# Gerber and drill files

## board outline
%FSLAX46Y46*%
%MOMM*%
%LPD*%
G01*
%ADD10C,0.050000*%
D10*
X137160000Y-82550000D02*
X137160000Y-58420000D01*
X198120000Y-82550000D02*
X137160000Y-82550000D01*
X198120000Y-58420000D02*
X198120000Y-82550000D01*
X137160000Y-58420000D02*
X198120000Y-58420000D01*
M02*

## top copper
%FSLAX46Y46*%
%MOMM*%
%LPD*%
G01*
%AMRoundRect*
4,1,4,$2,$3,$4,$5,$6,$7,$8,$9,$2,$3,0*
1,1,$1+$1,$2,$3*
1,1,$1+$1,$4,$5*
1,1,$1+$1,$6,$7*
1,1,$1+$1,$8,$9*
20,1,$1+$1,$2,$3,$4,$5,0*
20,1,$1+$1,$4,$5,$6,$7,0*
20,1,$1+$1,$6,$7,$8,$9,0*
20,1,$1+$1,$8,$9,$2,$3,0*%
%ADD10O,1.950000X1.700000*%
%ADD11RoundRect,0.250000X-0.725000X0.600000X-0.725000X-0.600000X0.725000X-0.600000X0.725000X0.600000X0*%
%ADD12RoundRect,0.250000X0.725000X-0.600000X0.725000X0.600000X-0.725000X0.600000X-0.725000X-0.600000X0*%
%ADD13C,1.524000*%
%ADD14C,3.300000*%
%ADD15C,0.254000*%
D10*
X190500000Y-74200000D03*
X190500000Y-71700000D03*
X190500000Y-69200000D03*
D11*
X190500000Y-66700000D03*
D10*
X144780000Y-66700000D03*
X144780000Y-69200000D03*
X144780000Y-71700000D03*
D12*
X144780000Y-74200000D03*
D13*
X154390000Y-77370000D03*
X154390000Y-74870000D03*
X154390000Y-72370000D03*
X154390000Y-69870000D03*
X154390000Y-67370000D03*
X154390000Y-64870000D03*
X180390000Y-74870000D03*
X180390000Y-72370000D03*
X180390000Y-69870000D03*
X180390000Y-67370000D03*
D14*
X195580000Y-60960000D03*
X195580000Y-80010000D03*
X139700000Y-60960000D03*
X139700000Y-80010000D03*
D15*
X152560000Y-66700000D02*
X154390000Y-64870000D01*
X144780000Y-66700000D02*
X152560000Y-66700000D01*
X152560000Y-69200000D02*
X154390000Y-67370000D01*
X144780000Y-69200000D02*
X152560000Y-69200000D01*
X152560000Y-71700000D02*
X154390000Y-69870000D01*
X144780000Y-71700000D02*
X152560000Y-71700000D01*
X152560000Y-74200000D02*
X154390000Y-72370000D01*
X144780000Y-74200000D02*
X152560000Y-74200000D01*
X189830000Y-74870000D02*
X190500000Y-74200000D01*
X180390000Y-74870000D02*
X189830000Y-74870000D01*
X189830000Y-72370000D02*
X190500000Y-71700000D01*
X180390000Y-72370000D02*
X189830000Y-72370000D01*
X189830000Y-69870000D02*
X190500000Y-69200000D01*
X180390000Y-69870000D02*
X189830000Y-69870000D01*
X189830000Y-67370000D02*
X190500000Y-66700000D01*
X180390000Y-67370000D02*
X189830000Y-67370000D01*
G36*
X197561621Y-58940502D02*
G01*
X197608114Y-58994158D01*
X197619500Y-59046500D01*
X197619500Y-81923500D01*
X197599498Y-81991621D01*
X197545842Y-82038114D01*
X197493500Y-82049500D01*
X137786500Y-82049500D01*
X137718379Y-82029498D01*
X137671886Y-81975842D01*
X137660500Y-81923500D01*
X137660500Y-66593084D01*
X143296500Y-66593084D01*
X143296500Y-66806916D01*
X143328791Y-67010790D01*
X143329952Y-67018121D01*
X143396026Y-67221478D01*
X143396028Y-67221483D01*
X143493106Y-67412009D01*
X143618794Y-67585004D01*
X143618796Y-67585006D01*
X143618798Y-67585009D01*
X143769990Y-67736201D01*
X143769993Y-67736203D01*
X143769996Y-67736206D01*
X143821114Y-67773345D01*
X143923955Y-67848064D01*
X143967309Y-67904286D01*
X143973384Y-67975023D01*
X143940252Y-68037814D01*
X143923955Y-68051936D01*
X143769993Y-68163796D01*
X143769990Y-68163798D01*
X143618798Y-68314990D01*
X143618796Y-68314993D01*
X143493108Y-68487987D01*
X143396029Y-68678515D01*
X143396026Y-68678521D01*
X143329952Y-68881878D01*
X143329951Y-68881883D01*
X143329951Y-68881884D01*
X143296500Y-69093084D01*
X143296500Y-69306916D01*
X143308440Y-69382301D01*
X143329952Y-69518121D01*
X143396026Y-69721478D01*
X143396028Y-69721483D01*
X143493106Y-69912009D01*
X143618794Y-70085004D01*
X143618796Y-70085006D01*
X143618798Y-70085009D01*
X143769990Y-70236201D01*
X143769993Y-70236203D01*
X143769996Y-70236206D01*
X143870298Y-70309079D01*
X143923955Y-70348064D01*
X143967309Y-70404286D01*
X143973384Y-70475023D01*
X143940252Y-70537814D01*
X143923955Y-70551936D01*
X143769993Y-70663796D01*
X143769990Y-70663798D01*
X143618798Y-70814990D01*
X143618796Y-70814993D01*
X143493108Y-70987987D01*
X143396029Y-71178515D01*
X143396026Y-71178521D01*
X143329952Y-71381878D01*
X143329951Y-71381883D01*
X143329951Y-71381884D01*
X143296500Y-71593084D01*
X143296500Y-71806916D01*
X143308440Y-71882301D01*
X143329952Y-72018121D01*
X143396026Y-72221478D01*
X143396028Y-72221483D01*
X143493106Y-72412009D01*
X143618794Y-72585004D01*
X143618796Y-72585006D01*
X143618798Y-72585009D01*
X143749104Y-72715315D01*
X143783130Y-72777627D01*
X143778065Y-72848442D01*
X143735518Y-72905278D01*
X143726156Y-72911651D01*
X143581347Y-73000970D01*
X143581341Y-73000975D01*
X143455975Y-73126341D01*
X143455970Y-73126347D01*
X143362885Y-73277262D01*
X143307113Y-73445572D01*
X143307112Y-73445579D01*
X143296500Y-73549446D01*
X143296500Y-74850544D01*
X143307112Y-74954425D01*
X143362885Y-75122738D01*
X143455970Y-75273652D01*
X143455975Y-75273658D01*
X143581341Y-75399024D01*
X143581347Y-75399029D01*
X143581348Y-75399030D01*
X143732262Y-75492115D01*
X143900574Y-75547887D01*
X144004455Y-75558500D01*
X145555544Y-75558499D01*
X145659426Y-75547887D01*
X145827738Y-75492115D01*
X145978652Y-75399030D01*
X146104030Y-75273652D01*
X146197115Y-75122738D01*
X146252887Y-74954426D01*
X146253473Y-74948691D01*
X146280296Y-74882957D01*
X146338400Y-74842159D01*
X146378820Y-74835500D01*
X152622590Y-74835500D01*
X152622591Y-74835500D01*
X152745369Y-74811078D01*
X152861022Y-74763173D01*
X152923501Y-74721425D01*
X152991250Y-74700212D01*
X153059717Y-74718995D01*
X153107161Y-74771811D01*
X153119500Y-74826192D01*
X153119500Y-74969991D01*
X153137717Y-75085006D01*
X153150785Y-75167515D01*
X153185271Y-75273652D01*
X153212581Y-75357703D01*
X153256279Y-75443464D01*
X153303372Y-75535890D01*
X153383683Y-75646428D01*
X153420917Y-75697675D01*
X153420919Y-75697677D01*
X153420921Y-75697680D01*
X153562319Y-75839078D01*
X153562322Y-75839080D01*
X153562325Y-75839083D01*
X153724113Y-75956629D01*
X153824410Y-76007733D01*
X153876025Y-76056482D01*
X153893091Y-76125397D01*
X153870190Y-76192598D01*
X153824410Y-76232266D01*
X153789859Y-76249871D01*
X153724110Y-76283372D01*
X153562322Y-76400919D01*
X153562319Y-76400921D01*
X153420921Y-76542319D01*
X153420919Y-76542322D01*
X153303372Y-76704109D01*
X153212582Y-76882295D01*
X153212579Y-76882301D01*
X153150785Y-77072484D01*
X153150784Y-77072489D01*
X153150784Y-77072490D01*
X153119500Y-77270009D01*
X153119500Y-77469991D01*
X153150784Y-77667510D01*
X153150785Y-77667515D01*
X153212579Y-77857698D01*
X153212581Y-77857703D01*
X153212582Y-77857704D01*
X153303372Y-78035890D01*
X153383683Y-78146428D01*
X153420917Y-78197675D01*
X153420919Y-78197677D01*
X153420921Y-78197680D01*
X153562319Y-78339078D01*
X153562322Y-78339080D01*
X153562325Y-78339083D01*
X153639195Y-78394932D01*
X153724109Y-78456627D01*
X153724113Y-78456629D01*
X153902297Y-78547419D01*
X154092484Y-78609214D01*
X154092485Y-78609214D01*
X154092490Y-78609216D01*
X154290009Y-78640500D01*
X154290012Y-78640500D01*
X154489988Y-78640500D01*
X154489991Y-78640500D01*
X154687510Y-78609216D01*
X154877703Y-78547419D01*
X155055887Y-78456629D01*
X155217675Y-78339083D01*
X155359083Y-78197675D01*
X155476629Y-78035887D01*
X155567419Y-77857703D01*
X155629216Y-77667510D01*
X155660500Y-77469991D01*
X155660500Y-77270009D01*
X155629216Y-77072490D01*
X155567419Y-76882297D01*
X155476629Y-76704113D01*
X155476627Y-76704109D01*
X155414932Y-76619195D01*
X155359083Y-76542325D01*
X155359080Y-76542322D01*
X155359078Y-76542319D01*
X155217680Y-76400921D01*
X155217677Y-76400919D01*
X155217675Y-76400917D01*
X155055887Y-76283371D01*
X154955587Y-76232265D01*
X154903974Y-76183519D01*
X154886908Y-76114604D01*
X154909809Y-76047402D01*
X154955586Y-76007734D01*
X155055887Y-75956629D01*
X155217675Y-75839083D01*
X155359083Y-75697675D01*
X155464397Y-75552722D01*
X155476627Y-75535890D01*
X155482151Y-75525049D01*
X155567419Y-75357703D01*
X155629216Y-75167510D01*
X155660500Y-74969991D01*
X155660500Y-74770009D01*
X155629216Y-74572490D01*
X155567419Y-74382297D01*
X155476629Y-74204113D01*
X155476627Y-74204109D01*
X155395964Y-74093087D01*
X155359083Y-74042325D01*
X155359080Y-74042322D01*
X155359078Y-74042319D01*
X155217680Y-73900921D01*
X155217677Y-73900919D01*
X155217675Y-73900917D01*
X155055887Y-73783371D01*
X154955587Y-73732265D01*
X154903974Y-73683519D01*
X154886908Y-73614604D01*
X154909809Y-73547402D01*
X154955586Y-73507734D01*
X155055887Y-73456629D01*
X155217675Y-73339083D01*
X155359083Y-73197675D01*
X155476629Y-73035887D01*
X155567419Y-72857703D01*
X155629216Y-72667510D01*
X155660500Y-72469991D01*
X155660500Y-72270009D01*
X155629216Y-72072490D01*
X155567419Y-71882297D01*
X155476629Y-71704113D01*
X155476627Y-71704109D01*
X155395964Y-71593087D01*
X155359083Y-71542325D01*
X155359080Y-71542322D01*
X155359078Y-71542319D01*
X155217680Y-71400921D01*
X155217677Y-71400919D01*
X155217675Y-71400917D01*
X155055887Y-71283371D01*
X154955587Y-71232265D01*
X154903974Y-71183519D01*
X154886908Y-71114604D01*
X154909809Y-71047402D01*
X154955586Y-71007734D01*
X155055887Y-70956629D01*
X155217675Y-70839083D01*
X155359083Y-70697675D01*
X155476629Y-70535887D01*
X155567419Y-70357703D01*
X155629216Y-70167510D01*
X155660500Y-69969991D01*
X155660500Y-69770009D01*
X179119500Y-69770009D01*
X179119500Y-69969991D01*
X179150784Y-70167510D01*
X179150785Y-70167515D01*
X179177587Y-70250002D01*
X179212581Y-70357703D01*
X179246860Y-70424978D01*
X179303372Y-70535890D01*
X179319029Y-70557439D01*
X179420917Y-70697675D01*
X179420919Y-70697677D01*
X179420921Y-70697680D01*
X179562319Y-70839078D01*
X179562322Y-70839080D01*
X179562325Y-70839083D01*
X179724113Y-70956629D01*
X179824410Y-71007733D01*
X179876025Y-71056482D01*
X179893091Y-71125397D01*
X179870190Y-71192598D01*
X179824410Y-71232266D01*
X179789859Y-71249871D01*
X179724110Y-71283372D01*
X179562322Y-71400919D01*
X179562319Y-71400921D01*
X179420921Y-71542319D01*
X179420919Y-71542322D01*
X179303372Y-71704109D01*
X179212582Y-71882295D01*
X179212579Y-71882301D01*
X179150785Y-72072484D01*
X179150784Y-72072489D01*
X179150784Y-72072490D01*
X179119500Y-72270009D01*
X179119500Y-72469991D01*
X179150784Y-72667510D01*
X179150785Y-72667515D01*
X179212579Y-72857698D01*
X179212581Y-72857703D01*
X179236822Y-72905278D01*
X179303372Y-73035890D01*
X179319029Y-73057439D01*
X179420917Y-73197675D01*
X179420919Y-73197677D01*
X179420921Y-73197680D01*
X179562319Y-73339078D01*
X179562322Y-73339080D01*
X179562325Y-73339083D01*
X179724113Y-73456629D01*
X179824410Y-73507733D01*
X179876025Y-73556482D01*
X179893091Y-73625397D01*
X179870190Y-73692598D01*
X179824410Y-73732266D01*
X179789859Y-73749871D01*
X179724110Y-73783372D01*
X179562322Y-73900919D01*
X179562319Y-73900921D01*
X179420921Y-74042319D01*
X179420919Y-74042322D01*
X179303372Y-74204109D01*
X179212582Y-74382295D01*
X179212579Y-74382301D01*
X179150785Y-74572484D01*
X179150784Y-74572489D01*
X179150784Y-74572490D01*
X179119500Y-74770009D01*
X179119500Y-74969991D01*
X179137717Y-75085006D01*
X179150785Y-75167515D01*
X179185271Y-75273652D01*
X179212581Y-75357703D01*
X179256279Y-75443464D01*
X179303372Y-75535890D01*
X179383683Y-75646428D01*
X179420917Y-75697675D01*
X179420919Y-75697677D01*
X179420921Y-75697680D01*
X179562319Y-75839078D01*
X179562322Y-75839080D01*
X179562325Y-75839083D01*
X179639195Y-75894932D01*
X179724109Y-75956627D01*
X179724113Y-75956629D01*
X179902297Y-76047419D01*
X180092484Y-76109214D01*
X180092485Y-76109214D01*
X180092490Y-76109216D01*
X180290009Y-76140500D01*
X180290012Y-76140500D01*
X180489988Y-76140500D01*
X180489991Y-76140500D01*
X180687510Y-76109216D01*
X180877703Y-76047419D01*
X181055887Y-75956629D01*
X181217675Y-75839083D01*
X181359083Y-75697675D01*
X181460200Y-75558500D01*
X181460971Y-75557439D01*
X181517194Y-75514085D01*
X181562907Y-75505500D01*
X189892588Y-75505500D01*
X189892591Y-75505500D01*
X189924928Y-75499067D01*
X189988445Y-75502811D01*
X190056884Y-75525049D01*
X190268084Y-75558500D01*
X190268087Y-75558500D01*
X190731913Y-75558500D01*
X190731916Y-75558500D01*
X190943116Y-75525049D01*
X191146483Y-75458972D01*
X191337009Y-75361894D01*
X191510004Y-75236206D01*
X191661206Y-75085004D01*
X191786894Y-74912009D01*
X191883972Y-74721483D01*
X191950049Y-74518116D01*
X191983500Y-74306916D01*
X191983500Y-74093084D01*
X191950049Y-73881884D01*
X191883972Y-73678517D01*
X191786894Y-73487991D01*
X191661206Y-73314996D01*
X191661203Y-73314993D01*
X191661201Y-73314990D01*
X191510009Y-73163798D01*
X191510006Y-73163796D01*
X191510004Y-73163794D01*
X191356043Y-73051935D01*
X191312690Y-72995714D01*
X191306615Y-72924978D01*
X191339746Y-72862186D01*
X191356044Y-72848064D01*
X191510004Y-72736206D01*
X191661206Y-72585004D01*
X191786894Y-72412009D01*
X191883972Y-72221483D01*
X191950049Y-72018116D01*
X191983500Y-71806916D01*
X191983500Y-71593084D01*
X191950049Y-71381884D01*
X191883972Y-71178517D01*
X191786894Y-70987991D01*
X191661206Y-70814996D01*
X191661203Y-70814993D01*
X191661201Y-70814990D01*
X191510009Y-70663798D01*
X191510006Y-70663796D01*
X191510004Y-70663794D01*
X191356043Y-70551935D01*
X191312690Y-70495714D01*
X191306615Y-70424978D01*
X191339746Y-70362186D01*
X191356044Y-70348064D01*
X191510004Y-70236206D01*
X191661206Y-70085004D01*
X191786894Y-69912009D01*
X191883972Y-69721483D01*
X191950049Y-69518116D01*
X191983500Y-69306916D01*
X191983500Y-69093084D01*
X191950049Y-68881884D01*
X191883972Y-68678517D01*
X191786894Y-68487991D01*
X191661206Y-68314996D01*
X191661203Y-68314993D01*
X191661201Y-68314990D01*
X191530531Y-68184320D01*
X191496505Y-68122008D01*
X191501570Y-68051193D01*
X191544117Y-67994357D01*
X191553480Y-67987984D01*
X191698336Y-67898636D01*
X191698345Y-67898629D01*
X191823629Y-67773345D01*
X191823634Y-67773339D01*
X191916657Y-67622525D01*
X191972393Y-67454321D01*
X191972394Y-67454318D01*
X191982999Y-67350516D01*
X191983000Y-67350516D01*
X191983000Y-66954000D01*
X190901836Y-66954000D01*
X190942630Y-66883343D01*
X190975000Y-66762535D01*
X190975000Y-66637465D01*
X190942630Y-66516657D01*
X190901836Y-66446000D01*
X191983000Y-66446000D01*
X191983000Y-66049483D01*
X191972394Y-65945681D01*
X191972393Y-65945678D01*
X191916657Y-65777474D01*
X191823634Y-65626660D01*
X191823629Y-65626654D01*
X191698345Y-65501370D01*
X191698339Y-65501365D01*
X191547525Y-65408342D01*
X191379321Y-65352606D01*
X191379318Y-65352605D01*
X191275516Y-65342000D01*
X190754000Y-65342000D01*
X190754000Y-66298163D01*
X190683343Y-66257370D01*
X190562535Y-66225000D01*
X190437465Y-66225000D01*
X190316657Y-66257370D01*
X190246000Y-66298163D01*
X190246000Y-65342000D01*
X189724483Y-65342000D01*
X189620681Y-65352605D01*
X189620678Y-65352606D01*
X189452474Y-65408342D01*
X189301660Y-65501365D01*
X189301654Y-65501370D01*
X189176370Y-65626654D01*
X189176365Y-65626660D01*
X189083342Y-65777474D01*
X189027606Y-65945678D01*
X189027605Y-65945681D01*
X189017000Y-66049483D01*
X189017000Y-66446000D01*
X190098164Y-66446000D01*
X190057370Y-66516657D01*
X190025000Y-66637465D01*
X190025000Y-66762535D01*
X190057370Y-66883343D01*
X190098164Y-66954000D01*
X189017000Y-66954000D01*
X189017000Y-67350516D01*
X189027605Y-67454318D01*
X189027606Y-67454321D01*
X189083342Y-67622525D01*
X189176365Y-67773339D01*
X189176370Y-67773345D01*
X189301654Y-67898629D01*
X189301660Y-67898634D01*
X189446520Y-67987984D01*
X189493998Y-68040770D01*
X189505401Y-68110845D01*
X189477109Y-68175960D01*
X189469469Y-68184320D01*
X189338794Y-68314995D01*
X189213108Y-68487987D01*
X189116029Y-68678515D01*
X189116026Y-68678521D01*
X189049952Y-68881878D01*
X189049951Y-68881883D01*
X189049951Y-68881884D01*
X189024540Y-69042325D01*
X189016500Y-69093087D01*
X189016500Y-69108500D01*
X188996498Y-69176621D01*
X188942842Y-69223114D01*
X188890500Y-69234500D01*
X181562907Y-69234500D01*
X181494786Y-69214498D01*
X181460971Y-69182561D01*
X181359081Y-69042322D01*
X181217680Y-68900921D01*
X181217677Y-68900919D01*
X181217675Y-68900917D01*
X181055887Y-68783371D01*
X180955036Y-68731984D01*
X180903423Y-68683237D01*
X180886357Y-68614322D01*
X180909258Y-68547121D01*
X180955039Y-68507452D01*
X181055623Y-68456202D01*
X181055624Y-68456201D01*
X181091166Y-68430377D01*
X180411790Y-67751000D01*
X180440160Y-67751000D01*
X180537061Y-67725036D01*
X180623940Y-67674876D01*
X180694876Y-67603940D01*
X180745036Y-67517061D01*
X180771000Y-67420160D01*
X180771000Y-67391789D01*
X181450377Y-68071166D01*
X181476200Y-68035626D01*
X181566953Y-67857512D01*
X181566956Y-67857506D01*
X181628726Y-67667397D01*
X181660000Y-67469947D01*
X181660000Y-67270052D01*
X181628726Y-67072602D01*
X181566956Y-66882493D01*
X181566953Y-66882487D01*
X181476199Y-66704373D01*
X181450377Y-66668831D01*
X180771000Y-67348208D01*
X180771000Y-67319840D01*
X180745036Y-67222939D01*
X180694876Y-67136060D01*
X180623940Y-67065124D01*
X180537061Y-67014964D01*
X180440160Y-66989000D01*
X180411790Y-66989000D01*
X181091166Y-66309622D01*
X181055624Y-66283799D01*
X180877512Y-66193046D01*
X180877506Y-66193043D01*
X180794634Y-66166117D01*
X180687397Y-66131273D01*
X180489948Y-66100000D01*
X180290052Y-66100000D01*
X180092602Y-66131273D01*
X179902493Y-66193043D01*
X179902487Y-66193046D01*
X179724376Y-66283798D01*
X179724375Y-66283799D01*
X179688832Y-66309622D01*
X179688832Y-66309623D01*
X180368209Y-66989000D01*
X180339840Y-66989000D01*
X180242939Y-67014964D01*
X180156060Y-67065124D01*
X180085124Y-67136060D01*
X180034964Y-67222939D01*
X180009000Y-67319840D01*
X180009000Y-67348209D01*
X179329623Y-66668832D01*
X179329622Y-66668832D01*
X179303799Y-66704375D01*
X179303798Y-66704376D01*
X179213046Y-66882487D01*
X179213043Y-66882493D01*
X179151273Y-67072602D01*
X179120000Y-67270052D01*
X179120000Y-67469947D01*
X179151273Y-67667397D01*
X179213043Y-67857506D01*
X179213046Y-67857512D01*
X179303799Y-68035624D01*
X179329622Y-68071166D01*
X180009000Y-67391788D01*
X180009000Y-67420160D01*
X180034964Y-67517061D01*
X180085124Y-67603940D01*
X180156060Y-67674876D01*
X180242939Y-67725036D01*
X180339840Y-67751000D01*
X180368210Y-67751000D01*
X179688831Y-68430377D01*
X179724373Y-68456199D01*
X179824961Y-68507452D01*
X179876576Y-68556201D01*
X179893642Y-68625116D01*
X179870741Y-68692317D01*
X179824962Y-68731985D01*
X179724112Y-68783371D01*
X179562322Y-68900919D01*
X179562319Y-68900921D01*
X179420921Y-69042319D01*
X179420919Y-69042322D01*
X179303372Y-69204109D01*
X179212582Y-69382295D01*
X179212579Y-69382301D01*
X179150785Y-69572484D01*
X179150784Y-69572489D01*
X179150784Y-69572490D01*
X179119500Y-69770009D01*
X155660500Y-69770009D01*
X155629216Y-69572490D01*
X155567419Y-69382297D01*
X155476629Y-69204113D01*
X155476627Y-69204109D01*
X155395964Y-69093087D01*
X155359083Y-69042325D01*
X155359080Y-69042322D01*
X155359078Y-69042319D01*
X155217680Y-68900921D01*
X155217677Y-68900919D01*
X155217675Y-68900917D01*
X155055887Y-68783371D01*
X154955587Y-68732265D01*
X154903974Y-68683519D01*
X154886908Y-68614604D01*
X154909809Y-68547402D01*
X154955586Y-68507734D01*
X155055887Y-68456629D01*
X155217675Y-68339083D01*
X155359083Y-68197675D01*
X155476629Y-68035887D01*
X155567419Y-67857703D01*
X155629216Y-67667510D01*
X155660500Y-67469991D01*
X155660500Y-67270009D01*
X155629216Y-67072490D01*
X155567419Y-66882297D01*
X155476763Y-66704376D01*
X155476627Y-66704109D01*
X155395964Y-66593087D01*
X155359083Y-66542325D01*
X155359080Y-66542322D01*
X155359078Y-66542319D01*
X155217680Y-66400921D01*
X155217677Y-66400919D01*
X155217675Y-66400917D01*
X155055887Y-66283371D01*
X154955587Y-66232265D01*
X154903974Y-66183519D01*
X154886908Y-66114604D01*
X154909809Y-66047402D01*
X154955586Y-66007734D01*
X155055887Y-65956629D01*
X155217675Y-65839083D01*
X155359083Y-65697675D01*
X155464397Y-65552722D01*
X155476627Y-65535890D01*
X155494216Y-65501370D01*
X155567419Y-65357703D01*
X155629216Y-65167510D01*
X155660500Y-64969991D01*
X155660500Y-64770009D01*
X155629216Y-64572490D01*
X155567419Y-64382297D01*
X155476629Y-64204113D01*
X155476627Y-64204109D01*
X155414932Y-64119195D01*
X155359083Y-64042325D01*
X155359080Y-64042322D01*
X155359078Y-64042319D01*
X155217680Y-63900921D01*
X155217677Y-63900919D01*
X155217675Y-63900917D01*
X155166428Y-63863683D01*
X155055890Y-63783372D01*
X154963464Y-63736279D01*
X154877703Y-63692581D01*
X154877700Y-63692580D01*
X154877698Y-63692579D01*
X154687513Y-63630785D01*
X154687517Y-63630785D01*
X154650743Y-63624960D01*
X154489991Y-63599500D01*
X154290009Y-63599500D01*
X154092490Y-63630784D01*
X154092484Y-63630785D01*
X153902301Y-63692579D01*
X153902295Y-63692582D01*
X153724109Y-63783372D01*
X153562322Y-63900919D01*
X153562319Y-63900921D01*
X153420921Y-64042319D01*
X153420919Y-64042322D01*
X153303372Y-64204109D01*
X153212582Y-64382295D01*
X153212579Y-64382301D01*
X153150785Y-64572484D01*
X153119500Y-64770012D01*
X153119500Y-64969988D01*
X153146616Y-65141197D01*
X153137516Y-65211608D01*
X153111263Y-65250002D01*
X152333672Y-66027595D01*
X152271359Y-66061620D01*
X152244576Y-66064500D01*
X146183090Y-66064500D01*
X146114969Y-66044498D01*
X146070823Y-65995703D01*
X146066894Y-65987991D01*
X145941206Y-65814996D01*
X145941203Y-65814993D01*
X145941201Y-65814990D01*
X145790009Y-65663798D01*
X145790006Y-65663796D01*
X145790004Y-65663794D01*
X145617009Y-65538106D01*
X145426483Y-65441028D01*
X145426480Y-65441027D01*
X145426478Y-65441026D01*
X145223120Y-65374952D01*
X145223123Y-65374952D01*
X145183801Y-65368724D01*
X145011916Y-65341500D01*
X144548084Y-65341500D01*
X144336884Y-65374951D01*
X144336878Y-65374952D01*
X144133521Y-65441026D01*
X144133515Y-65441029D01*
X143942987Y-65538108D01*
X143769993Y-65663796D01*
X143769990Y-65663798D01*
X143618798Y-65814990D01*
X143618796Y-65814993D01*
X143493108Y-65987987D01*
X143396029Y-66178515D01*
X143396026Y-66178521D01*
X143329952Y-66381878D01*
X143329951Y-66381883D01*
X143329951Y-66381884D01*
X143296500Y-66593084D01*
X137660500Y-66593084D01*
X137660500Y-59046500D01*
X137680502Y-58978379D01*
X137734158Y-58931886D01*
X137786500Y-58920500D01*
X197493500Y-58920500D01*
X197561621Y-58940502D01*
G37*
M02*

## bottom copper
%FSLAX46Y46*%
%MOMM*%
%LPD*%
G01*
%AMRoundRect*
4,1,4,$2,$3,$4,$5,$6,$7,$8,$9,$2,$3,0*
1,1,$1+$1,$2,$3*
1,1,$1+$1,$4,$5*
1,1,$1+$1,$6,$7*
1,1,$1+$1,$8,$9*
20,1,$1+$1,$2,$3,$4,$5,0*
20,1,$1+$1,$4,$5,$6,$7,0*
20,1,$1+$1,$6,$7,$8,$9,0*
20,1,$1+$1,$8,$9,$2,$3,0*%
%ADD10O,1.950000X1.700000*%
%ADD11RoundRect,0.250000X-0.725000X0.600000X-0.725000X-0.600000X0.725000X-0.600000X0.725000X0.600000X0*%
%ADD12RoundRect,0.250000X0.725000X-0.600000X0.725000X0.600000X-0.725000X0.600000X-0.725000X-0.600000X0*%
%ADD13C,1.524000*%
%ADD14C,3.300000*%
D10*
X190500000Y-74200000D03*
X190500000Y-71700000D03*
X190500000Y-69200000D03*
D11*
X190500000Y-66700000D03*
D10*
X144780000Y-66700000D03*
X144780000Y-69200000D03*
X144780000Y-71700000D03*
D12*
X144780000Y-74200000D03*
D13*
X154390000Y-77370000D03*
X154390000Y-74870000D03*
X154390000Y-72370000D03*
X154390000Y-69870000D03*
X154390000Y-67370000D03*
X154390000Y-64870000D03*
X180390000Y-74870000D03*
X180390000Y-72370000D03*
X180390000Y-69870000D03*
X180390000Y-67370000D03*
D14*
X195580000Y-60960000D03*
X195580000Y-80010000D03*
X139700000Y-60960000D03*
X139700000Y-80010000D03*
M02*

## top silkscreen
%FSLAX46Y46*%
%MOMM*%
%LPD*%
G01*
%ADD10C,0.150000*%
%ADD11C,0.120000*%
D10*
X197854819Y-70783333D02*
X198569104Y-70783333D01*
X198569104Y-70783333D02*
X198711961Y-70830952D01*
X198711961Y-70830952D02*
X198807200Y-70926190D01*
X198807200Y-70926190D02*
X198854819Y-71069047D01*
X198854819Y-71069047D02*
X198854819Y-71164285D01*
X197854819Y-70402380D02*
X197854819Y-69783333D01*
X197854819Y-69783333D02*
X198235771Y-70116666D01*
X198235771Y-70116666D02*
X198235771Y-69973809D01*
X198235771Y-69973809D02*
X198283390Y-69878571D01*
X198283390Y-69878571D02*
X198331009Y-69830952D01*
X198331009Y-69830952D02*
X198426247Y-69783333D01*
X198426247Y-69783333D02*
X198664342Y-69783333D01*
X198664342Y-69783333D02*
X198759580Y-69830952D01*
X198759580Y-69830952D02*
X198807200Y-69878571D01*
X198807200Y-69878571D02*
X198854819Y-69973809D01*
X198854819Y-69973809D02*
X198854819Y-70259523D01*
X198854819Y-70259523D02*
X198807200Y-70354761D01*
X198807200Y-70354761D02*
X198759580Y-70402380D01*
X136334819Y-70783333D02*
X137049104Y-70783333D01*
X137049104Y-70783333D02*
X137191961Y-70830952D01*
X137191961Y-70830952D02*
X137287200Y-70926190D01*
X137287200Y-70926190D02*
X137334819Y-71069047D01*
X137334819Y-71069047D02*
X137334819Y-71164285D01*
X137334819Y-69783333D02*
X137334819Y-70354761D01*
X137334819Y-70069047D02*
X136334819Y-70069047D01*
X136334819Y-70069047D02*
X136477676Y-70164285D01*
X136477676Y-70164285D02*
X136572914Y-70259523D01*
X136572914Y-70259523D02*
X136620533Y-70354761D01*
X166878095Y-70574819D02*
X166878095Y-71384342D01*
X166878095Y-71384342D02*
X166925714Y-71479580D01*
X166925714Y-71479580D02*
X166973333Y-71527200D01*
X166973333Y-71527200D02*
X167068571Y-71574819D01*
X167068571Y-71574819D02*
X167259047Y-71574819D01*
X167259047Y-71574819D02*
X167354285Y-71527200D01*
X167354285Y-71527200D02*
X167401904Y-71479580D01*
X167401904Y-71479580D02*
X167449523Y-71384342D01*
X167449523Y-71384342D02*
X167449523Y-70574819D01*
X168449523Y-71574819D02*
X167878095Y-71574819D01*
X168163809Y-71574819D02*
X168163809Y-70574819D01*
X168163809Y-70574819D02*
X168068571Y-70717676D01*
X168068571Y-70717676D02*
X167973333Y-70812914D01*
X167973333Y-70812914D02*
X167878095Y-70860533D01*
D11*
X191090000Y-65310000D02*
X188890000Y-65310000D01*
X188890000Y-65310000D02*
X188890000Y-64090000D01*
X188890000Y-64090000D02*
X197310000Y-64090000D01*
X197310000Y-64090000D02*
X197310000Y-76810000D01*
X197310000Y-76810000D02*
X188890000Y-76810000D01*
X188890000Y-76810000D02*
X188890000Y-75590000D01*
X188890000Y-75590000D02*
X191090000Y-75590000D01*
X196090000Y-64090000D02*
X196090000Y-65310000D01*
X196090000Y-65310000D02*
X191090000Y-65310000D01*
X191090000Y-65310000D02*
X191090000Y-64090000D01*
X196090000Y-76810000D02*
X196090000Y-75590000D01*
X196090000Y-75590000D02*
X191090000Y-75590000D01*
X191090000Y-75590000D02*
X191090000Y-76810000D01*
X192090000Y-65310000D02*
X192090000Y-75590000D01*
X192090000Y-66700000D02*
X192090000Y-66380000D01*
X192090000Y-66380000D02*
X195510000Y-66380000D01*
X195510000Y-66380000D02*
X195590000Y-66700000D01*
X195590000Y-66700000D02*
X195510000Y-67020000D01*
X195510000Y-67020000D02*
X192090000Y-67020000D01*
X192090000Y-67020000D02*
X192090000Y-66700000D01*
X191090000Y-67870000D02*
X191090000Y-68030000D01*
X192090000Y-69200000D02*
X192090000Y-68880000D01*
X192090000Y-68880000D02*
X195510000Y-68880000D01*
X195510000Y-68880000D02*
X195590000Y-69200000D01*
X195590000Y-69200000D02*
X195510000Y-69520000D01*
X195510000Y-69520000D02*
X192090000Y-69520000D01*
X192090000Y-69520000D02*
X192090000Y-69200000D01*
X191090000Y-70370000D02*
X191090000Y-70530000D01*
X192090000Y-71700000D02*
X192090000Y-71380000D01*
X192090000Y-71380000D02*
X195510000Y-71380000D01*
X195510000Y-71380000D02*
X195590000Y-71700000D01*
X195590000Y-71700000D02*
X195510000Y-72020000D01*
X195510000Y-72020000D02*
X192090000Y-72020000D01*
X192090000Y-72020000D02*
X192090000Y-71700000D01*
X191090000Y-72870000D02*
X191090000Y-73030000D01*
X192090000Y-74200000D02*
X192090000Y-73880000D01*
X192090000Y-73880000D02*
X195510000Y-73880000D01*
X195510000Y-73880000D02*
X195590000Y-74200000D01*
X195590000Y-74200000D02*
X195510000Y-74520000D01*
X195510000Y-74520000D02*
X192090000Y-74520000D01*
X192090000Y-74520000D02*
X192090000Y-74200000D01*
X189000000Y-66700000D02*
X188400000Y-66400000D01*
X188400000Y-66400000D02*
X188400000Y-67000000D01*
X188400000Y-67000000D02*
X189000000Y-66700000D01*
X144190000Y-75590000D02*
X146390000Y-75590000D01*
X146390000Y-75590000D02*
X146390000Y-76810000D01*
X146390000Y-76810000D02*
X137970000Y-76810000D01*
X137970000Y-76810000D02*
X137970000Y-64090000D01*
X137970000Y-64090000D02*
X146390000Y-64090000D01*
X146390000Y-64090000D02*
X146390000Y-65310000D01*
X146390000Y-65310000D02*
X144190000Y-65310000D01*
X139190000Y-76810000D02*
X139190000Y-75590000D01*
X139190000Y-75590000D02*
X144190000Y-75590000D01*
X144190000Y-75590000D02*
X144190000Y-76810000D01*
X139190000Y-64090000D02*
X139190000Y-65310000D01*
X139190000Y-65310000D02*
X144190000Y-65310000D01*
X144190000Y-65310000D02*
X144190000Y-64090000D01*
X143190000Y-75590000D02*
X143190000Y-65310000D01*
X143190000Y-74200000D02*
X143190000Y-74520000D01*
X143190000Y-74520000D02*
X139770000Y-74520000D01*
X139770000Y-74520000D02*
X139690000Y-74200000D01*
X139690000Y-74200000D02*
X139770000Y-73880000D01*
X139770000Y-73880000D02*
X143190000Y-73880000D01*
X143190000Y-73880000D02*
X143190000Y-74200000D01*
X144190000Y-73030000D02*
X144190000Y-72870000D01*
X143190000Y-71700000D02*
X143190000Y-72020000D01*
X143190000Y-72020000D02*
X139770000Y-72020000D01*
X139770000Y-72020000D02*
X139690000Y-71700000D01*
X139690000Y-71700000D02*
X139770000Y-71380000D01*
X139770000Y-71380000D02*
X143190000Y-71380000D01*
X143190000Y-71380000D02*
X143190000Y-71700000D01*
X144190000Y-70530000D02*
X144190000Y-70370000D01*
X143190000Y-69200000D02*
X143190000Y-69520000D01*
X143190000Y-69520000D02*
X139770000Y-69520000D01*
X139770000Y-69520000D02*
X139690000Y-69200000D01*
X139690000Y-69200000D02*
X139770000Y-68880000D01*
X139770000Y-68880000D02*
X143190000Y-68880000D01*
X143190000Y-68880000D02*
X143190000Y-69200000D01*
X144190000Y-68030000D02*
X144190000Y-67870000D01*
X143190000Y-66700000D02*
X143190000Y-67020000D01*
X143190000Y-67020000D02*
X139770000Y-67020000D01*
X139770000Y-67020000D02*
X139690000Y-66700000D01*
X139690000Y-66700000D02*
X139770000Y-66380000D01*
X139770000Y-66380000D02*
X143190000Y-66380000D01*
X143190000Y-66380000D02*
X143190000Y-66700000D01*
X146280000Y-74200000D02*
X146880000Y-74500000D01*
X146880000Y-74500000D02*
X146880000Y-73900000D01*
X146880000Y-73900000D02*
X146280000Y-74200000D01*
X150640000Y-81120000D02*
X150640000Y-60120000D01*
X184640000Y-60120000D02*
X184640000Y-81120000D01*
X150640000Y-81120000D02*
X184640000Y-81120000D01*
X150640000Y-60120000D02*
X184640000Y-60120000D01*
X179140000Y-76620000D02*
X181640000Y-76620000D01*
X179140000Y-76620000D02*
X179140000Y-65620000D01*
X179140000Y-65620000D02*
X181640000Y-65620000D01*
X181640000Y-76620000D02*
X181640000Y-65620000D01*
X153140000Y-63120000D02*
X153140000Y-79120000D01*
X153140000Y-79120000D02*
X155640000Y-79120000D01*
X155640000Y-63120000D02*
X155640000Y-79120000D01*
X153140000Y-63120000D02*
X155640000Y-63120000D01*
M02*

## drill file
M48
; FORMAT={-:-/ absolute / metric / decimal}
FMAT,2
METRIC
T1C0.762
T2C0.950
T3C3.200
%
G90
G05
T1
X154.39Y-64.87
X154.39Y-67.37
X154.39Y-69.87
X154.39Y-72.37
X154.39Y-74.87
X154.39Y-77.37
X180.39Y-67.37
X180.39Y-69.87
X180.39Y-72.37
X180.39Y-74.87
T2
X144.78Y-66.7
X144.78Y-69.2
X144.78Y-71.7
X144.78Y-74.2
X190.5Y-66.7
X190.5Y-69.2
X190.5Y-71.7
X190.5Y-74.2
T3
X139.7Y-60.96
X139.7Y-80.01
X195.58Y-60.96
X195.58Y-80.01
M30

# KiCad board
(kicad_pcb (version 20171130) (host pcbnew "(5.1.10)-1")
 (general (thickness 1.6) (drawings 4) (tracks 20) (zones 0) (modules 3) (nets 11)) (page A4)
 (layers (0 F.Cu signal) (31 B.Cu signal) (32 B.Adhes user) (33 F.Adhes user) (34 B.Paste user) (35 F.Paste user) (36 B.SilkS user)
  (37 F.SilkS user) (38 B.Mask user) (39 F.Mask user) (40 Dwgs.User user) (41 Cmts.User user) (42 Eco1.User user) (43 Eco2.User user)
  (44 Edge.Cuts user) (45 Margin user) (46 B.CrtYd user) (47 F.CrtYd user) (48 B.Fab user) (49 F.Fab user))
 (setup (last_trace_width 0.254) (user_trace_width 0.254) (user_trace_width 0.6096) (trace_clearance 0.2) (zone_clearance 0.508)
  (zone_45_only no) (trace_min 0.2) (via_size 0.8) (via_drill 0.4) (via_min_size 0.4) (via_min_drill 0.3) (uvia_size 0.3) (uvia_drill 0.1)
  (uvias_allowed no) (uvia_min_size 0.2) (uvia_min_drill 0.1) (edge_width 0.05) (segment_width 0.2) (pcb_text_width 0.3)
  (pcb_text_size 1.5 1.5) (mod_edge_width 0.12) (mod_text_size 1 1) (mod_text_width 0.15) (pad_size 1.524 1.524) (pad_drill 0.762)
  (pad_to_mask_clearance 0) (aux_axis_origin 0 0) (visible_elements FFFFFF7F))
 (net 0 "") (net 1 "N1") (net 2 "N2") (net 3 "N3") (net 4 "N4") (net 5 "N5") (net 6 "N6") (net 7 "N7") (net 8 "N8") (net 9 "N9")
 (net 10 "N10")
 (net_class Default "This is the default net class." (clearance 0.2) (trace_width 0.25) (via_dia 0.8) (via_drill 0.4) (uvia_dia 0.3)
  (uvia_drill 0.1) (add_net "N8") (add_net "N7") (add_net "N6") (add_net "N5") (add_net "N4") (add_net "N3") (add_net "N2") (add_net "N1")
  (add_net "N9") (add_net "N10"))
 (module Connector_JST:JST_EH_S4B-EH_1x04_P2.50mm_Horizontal (layer F.Cu) (at 190.5 66.7 270)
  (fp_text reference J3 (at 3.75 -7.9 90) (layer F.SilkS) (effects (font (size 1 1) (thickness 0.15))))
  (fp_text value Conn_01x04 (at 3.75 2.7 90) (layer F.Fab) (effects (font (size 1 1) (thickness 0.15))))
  (fp_line (start -1.39 -0.59) (end -1.39 1.61) (layer F.SilkS) (width 0.12))
  (fp_line (start -1.39 1.61) (end -2.61 1.61) (layer F.SilkS) (width 0.12))
  (fp_line (start -2.61 1.61) (end -2.61 -6.81) (layer F.SilkS) (width 0.12))
  (fp_line (start -2.61 -6.81) (end 10.11 -6.81) (layer F.SilkS) (width 0.12))
  (fp_line (start 10.11 -6.81) (end 10.11 1.61) (layer F.SilkS) (width 0.12))
  (fp_line (start 10.11 1.61) (end 8.89 1.61) (layer F.SilkS) (width 0.12))
  (fp_line (start 8.89 1.61) (end 8.89 -0.59) (layer F.SilkS) (width 0.12))
  (fp_line (start -2.61 -5.59) (end -1.39 -5.59) (layer F.SilkS) (width 0.12))
  (fp_line (start -1.39 -5.59) (end -1.39 -0.59) (layer F.SilkS) (width 0.12))
  (fp_line (start -1.39 -0.59) (end -2.61 -0.59) (layer F.SilkS) (width 0.12))
  (fp_line (start 10.11 -5.59) (end 8.89 -5.59) (layer F.SilkS) (width 0.12))
  (fp_line (start 8.89 -5.59) (end 8.89 -0.59) (layer F.SilkS) (width 0.12))
  (fp_line (start 8.89 -0.59) (end 10.11 -0.59) (layer F.SilkS) (width 0.12))
  (fp_line (start -1.39 -1.59) (end 8.89 -1.59) (layer F.SilkS) (width 0.12))
  (fp_line (start 0 -1.59) (end -0.32 -1.59) (layer F.SilkS) (width 0.12))
  (fp_line (start -0.32 -1.59) (end -0.32 -5.01) (layer F.SilkS) (width 0.12))
  (fp_line (start -0.32 -5.01) (end 0 -5.09) (layer F.SilkS) (width 0.12))
  (fp_line (start 0 -5.09) (end 0.32 -5.01) (layer F.SilkS) (width 0.12))
  (fp_line (start 0.32 -5.01) (end 0.32 -1.59) (layer F.SilkS) (width 0.12))
  (fp_line (start 0.32 -1.59) (end 0 -1.59) (layer F.SilkS) (width 0.12))
  (fp_line (start 1.17 -0.59) (end 1.33 -0.59) (layer F.SilkS) (width 0.12))
  (fp_line (start 2.5 -1.59) (end 2.18 -1.59) (layer F.SilkS) (width 0.12))
  (fp_line (start 2.18 -1.59) (end 2.18 -5.01) (layer F.SilkS) (width 0.12))
  (fp_line (start 2.18 -5.01) (end 2.5 -5.09) (layer F.SilkS) (width 0.12))
  (fp_line (start 2.5 -5.09) (end 2.82 -5.01) (layer F.SilkS) (width 0.12))
  (fp_line (start 2.82 -5.01) (end 2.82 -1.59) (layer F.SilkS) (width 0.12))
  (fp_line (start 2.82 -1.59) (end 2.5 -1.59) (layer F.SilkS) (width 0.12))
  (fp_line (start 3.67 -0.59) (end 3.83 -0.59) (layer F.SilkS) (width 0.12))
  (fp_line (start 5 -1.59) (end 4.68 -1.59) (layer F.SilkS) (width 0.12))
  (fp_line (start 4.68 -1.59) (end 4.68 -5.01) (layer F.SilkS) (width 0.12))
  (fp_line (start 4.68 -5.01) (end 5 -5.09) (layer F.SilkS) (width 0.12))
  (fp_line (start 5 -5.09) (end 5.32 -5.01) (layer F.SilkS) (width 0.12))
  (fp_line (start 5.32 -5.01) (end 5.32 -1.59) (layer F.SilkS) (width 0.12))
  (fp_line (start 5.32 -1.59) (end 5 -1.59) (layer F.SilkS) (width 0.12))
  (fp_line (start 6.17 -0.59) (end 6.33 -0.59) (layer F.SilkS) (width 0.12))
  (fp_line (start 7.5 -1.59) (end 7.18 -1.59) (layer F.SilkS) (width 0.12))
  (fp_line (start 7.18 -1.59) (end 7.18 -5.01) (layer F.SilkS) (width 0.12))
  (fp_line (start 7.18 -5.01) (end 7.5 -5.09) (layer F.SilkS) (width 0.12))
  (fp_line (start 7.5 -5.09) (end 7.82 -5.01) (layer F.SilkS) (width 0.12))
  (fp_line (start 7.82 -5.01) (end 7.82 -1.59) (layer F.SilkS) (width 0.12))
  (fp_line (start 7.82 -1.59) (end 7.5 -1.59) (layer F.SilkS) (width 0.12))
  (fp_line (start 0 1.5) (end -0.3 2.1) (layer F.SilkS) (width 0.12))
  (fp_line (start -0.3 2.1) (end 0.3 2.1) (layer F.SilkS) (width 0.12))
  (fp_line (start 0.3 2.1) (end 0 1.5) (layer F.SilkS) (width 0.12))
  (pad 4 thru_hole oval (at 7.5 0 270) (size 1.7 1.95) (drill 0.95) (layers *.Cu *.Mask) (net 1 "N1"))
  (pad 3 thru_hole oval (at 5 0 270) (size 1.7 1.95) (drill 0.95) (layers *.Cu *.Mask) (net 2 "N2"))
  (pad 2 thru_hole oval (at 2.5 0 270) (size 1.7 1.95) (drill 0.95) (layers *.Cu *.Mask) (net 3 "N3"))
  (pad 1 thru_hole roundrect (at 0 0 270) (size 1.7 1.95) (drill 0.95) (layers *.Cu *.Mask) (roundrect_rratio 0.147059) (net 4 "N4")))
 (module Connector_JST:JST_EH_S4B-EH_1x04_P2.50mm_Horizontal (layer F.Cu) (at 144.78 74.2 90)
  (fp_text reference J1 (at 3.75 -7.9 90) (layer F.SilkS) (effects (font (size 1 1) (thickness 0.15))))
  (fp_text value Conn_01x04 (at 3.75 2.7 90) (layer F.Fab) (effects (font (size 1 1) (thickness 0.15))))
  (fp_line (start -1.39 -0.59) (end -1.39 1.61) (layer F.SilkS) (width 0.12))
  (fp_line (start -1.39 1.61) (end -2.61 1.61) (layer F.SilkS) (width 0.12))
  (fp_line (start -2.61 1.61) (end -2.61 -6.81) (layer F.SilkS) (width 0.12))
  (fp_line (start -2.61 -6.81) (end 10.11 -6.81) (layer F.SilkS) (width 0.12))
  (fp_line (start 10.11 -6.81) (end 10.11 1.61) (layer F.SilkS) (width 0.12))
  (fp_line (start 10.11 1.61) (end 8.89 1.61) (layer F.SilkS) (width 0.12))
  (fp_line (start 8.89 1.61) (end 8.89 -0.59) (layer F.SilkS) (width 0.12))
  (fp_line (start -2.61 -5.59) (end -1.39 -5.59) (layer F.SilkS) (width 0.12))
  (fp_line (start -1.39 -5.59) (end -1.39 -0.59) (layer F.SilkS) (width 0.12))
  (fp_line (start -1.39 -0.59) (end -2.61 -0.59) (layer F.SilkS) (width 0.12))
  (fp_line (start 10.11 -5.59) (end 8.89 -5.59) (layer F.SilkS) (width 0.12))
  (fp_line (start 8.89 -5.59) (end 8.89 -0.59) (layer F.SilkS) (width 0.12))
  (fp_line (start 8.89 -0.59) (end 10.11 -0.59) (layer F.SilkS) (width 0.12))
  (fp_line (start -1.39 -1.59) (end 8.89 -1.59) (layer F.SilkS) (width 0.12))
  (fp_line (start 0 -1.59) (end -0.32 -1.59) (layer F.SilkS) (width 0.12))
  (fp_line (start -0.32 -1.59) (end -0.32 -5.01) (layer F.SilkS) (width 0.12))
  (fp_line (start -0.32 -5.01) (end 0 -5.09) (layer F.SilkS) (width 0.12))
  (fp_line (start 0 -5.09) (end 0.32 -5.01) (layer F.SilkS) (width 0.12))
  (fp_line (start 0.32 -5.01) (end 0.32 -1.59) (layer F.SilkS) (width 0.12))
  (fp_line (start 0.32 -1.59) (end 0 -1.59) (layer F.SilkS) (width 0.12))
  (fp_line (start 1.17 -0.59) (end 1.33 -0.59) (layer F.SilkS) (width 0.12))
  (fp_line (start 2.5 -1.59) (end 2.18 -1.59) (layer F.SilkS) (width 0.12))
  (fp_line (start 2.18 -1.59) (end 2.18 -5.01) (layer F.SilkS) (width 0.12))
  (fp_line (start 2.18 -5.01) (end 2.5 -5.09) (layer F.SilkS) (width 0.12))
  (fp_line (start 2.5 -5.09) (end 2.82 -5.01) (layer F.SilkS) (width 0.12))
  (fp_line (start 2.82 -5.01) (end 2.82 -1.59) (layer F.SilkS) (width 0.12))
  (fp_line (start 2.82 -1.59) (end 2.5 -1.59) (layer F.SilkS) (width 0.12))
  (fp_line (start 3.67 -0.59) (end 3.83 -0.59) (layer F.SilkS) (width 0.12))
  (fp_line (start 5 -1.59) (end 4.68 -1.59) (layer F.SilkS) (width 0.12))
  (fp_line (start 4.68 -1.59) (end 4.68 -5.01) (layer F.SilkS) (width 0.12))
  (fp_line (start 4.68 -5.01) (end 5 -5.09) (layer F.SilkS) (width 0.12))
  (fp_line (start 5 -5.09) (end 5.32 -5.01) (layer F.SilkS) (width 0.12))
  (fp_line (start 5.32 -5.01) (end 5.32 -1.59) (layer F.SilkS) (width 0.12))
  (fp_line (start 5.32 -1.59) (end 5 -1.59) (layer F.SilkS) (width 0.12))
  (fp_line (start 6.17 -0.59) (end 6.33 -0.59) (layer F.SilkS) (width 0.12))
  (fp_line (start 7.5 -1.59) (end 7.18 -1.59) (layer F.SilkS) (width 0.12))
  (fp_line (start 7.18 -1.59) (end 7.18 -5.01) (layer F.SilkS) (width 0.12))
  (fp_line (start 7.18 -5.01) (end 7.5 -5.09) (layer F.SilkS) (width 0.12))
  (fp_line (start 7.5 -5.09) (end 7.82 -5.01) (layer F.SilkS) (width 0.12))
  (fp_line (start 7.82 -5.01) (end 7.82 -1.59) (layer F.SilkS) (width 0.12))
  (fp_line (start 7.82 -1.59) (end 7.5 -1.59) (layer F.SilkS) (width 0.12))
  (fp_line (start 0 1.5) (end -0.3 2.1) (layer F.SilkS) (width 0.12))
  (fp_line (start -0.3 2.1) (end 0.3 2.1) (layer F.SilkS) (width 0.12))
  (fp_line (start 0.3 2.1) (end 0 1.5) (layer F.SilkS) (width 0.12))
  (pad 4 thru_hole oval (at 7.5 0 90) (size 1.7 1.95) (drill 0.95) (layers *.Cu *.Mask) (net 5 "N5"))
  (pad 3 thru_hole oval (at 5 0 90) (size 1.7 1.95) (drill 0.95) (layers *.Cu *.Mask) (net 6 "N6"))
  (pad 2 thru_hole oval (at 2.5 0 90) (size 1.7 1.95) (drill 0.95) (layers *.Cu *.Mask) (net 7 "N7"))
  (pad 1 thru_hole roundrect (at 0 0 90) (size 1.7 1.95) (drill 0.95) (layers *.Cu *.Mask) (roundrect_rratio 0.147059) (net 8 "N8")))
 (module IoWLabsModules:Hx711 (layer F.Cu) (at 167.64 71.12)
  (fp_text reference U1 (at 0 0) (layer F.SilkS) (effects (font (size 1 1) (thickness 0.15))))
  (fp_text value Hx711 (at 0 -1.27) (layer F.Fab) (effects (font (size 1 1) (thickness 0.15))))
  (fp_line (start -17 10) (end -17 -11) (layer F.SilkS) (width 0.12))
  (fp_line (start 17 -11) (end 17 10) (layer F.SilkS) (width 0.12))
  (fp_line (start -17 10) (end 17 10) (layer F.SilkS) (width 0.12))
  (fp_line (start -17 -11) (end 17 -11) (layer F.SilkS) (width 0.12))
  (fp_line (start 11.5 5.5) (end 14 5.5) (layer F.SilkS) (width 0.12))
  (fp_line (start 11.5 5.5) (end 11.5 -5.5) (layer F.SilkS) (width 0.12))
  (fp_line (start 11.5 -5.5) (end 14 -5.5) (layer F.SilkS) (width 0.12))
  (fp_line (start 14 5.5) (end 14 -5.5) (layer F.SilkS) (width 0.12))
  (fp_line (start -14.5 -8) (end -14.5 8) (layer F.SilkS) (width 0.12))
  (fp_line (start -14.5 8) (end -12 8) (layer F.SilkS) (width 0.12))
  (fp_line (start -12 -8) (end -12 8) (layer F.SilkS) (width 0.12))
  (fp_line (start -14.5 -8) (end -12 -8) (layer F.SilkS) (width 0.12))
  (pad 10 thru_hole circle (at -13.25 6.25) (size 1.524 1.524) (drill 0.762) (layers *.Cu *.Mask) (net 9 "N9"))
  (pad 9 thru_hole circle (at -13.25 3.75) (size 1.524 1.524) (drill 0.762) (layers *.Cu *.Mask) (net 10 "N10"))
  (pad 4 thru_hole circle (at -13.25 1.25) (size 1.524 1.524) (drill 0.762) (layers *.Cu *.Mask) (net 8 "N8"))
  (pad 3 thru_hole circle (at -13.25 -1.25) (size 1.524 1.524) (drill 0.762) (layers *.Cu *.Mask) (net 7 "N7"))
  (pad 2 thru_hole circle (at -13.25 -3.75) (size 1.524 1.524) (drill 0.762) (layers *.Cu *.Mask) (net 6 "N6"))
  (pad 1 thru_hole circle (at -13.25 -6.25) (size 1.524 1.524) (drill 0.762) (layers *.Cu *.Mask) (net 5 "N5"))
  (pad 8 thru_hole circle (at 12.75 3.75) (size 1.524 1.524) (drill 0.762) (layers *.Cu *.Mask) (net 1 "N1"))
  (pad 7 thru_hole circle (at 12.75 1.25) (size 1.524 1.524) (drill 0.762) (layers *.Cu *.Mask) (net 2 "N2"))
  (pad 6 thru_hole circle (at 12.75 -1.25) (size 1.524 1.524) (drill 0.762) (layers *.Cu *.Mask) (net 3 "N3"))
  (pad 5 thru_hole circle (at 12.75 -3.75) (size 1.524 1.524) (drill 0.762) (layers *.Cu *.Mask) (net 4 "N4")))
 (gr_line (start 137.16 82.55) (end 137.16 58.42) (layer Edge.Cuts) (width 0.05))
 (gr_line (start 198.12 82.55) (end 137.16 82.55) (layer Edge.Cuts) (width 0.05))
 (gr_line (start 198.12 58.42) (end 198.12 82.55) (layer Edge.Cuts) (width 0.05))
 (gr_line (start 137.16 58.42) (end 198.12 58.42) (layer Edge.Cuts) (width 0.05))
 (via (at 195.58 60.96) (size 3.3) (drill 3.2) (layers F.Cu B.Cu) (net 4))
 (via (at 195.58 80.01) (size 3.3) (drill 3.2) (layers F.Cu B.Cu) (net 4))
 (via (at 139.7 60.96) (size 3.3) (drill 3.2) (layers F.Cu B.Cu) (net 4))
 (via (at 139.7 80.01) (size 3.3) (drill 3.2) (layers F.Cu B.Cu) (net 4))
 (segment (start 152.56 66.7) (end 154.39 64.87) (width 0.254) (layer F.Cu) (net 5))
 (segment (start 144.78 66.7) (end 152.56 66.7) (width 0.254) (layer F.Cu) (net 5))
 (segment (start 152.56 69.2) (end 154.39 67.37) (width 0.254) (layer F.Cu) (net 6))
 (segment (start 144.78 69.2) (end 152.56 69.2) (width 0.254) (layer F.Cu) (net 6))
 (segment (start 152.56 71.7) (end 154.39 69.87) (width 0.254) (layer F.Cu) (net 7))
 (segment (start 144.78 71.7) (end 152.56 71.7) (width 0.254) (layer F.Cu) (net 7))
 (segment (start 152.56 74.2) (end 154.39 72.37) (width 0.254) (layer F.Cu) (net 8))
 (segment (start 144.78 74.2) (end 152.56 74.2) (width 0.254) (layer F.Cu) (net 8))
 (segment (start 189.83 74.87) (end 190.5 74.2) (width 0.254) (layer F.Cu) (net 1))
 (segment (start 180.39 74.87) (end 189.83 74.87) (width 0.254) (layer F.Cu) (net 1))
 (segment (start 189.83 72.37) (end 190.5 71.7) (width 0.254) (layer F.Cu) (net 2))
 (segment (start 180.39 72.37) (end 189.83 72.37) (width 0.254) (layer F.Cu) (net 2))
 (segment (start 189.83 69.87) (end 190.5 69.2) (width 0.254) (layer F.Cu) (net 3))
 (segment (start 180.39 69.87) (end 189.83 69.87) (width 0.254) (layer F.Cu) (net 3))
 (segment (start 189.83 67.37) (end 190.5 66.7) (width 0.254) (layer F.Cu) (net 4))
 (segment (start 180.39 67.37) (end 189.83 67.37) (width 0.254) (layer F.Cu) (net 4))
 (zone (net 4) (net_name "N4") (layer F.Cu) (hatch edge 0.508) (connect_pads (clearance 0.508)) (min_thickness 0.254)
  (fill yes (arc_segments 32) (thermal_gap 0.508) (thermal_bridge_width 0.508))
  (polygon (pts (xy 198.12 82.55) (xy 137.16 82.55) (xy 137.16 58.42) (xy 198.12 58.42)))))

